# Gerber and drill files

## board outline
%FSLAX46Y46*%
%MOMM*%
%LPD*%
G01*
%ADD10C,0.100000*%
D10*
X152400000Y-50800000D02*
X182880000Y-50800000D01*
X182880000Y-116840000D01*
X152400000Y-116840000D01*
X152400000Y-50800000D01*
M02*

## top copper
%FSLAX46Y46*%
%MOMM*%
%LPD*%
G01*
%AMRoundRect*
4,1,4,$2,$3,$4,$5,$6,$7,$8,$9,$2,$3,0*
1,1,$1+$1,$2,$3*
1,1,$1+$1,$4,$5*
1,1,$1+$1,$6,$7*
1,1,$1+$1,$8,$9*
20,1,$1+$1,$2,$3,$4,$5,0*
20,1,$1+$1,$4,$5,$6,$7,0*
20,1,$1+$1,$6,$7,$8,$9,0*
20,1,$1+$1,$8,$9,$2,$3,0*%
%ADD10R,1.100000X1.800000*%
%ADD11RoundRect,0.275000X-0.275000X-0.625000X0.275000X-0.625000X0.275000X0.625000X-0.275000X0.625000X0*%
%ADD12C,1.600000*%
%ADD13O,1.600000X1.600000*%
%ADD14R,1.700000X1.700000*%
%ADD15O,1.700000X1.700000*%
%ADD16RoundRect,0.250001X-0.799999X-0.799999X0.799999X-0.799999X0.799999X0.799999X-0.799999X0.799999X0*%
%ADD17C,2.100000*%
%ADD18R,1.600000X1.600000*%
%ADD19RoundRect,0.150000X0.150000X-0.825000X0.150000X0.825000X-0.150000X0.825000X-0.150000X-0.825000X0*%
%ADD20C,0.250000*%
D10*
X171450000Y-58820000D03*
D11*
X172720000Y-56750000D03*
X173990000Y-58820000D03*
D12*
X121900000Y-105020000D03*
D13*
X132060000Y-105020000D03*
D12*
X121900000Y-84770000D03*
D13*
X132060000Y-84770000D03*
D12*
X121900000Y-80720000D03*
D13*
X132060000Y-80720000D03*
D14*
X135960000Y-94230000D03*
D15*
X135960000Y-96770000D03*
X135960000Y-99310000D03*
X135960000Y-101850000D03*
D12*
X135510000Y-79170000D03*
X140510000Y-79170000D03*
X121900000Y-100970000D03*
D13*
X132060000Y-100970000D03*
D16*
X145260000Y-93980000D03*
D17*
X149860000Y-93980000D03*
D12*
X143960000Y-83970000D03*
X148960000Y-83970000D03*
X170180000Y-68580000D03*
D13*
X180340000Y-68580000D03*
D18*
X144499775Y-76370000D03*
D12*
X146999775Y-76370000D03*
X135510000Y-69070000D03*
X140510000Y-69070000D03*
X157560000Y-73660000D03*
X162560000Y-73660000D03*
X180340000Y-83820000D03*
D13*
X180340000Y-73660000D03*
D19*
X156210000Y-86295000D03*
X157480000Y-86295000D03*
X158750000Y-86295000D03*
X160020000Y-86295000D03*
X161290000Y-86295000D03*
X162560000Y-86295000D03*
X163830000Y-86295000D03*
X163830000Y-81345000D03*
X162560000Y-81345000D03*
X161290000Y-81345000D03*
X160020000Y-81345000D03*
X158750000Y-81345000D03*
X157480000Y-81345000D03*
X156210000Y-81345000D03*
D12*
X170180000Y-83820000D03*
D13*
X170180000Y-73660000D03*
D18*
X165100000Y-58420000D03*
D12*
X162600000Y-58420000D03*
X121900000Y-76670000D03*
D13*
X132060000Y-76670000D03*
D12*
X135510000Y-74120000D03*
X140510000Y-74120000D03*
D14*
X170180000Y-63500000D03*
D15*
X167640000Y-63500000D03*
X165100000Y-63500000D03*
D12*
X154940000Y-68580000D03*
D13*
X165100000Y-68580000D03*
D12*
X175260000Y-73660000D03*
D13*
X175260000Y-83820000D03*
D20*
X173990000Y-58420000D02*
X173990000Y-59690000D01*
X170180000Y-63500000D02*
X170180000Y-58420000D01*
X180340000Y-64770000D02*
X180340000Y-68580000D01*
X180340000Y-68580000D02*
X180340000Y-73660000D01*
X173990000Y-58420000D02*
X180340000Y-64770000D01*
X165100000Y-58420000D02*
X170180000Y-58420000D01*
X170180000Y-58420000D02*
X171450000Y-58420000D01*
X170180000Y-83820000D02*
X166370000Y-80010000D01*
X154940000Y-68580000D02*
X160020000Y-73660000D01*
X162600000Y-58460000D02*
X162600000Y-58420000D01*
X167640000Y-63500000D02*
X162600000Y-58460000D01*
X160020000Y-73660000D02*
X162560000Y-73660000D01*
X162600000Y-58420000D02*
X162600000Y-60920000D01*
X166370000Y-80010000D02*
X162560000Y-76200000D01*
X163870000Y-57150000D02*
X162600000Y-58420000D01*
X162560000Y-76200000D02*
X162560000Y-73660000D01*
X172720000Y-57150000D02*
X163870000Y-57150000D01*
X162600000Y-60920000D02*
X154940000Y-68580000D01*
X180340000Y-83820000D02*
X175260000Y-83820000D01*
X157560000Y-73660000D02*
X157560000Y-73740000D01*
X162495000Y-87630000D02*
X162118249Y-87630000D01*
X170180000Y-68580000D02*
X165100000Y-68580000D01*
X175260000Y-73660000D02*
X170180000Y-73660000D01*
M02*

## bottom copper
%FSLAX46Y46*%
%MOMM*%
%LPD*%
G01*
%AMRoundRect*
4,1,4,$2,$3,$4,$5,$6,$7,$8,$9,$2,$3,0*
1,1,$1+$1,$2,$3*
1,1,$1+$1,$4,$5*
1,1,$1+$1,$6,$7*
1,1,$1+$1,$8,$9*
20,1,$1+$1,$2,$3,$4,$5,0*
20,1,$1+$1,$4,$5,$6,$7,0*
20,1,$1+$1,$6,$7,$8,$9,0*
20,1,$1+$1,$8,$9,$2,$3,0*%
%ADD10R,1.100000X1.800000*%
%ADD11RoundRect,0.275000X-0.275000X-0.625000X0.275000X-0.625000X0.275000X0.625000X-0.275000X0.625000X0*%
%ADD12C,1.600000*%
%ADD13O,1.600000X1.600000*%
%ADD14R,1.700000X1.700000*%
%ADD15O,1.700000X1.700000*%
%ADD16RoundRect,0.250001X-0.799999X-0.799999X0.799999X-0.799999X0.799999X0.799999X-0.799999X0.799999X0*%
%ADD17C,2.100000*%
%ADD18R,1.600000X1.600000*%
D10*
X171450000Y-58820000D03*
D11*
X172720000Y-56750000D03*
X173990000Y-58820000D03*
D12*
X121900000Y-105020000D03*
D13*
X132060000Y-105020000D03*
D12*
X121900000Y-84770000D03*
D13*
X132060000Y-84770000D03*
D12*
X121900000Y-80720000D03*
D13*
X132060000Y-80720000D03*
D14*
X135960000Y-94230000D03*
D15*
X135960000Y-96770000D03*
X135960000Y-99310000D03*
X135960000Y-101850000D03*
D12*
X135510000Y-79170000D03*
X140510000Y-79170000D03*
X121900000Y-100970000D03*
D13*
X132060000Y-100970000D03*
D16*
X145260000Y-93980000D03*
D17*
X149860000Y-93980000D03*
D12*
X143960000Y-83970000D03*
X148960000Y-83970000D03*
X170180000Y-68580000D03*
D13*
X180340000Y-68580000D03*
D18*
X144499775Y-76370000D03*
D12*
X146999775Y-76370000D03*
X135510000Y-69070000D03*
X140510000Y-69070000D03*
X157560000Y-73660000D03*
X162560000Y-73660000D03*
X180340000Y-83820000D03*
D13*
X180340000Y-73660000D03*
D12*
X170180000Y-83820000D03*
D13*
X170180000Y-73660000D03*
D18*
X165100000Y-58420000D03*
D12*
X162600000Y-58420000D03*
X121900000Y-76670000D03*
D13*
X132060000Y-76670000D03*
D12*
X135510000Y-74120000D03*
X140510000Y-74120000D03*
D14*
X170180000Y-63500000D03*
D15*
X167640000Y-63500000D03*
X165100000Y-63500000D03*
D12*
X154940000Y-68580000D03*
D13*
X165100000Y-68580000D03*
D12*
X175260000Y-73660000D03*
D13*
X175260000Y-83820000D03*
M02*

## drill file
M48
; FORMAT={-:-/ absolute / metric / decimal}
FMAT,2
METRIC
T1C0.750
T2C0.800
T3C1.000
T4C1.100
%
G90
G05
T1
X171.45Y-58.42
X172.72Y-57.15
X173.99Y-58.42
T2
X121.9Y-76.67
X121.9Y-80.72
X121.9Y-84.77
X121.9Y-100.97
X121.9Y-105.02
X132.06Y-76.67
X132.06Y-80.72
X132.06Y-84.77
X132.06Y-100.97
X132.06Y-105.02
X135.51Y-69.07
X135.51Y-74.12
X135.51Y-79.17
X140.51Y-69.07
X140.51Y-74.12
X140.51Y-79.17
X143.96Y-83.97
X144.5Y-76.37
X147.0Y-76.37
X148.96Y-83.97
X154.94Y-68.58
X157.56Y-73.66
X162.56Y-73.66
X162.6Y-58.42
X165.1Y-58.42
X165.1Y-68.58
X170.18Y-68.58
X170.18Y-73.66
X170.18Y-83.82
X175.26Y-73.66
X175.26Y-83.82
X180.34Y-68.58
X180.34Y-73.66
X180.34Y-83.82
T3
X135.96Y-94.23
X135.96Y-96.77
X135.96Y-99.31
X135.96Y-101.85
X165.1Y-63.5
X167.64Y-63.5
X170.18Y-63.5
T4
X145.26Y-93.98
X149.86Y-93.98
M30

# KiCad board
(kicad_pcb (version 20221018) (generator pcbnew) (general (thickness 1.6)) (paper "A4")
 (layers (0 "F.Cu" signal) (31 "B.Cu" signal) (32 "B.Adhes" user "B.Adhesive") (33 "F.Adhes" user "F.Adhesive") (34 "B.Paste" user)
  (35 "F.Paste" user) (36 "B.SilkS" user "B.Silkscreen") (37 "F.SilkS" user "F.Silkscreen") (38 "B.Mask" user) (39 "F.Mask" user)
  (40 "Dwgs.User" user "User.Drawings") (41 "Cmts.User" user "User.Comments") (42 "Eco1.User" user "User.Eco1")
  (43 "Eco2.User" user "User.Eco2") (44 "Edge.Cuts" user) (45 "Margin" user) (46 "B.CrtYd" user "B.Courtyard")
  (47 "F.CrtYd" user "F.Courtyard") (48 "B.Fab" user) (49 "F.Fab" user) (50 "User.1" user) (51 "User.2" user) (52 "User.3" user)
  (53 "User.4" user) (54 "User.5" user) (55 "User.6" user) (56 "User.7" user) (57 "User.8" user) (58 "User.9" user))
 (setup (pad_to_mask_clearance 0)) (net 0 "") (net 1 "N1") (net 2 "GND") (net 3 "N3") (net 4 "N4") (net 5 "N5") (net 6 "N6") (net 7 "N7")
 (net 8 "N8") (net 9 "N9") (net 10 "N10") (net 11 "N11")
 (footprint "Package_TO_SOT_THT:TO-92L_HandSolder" (layer "F.Cu") (at 171.45 58.42)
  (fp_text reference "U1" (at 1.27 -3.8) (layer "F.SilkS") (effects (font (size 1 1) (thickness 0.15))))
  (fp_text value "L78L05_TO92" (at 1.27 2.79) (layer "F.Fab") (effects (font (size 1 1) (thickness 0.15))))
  (pad "1" thru_hole rect (at 0 0) (size 1.1 1.8) (drill 0.75 (offset 0 0.4)) (layers "*.Cu" "*.Mask") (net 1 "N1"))
  (pad "2" thru_hole roundrect (at 1.27 -1.27) (size 1.1 1.8) (drill 0.75 (offset 0 -0.4)) (layers "*.Cu" "*.Mask") (roundrect_rratio 0.25)
   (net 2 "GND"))
  (pad "3" thru_hole roundrect (at 2.54 0) (size 1.1 1.8) (drill 0.75 (offset 0 0.4)) (layers "*.Cu" "*.Mask") (roundrect_rratio 0.25)
   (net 1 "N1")))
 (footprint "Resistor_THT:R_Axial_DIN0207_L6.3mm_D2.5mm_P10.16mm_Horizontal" (layer "F.Cu") (at 121.9 105.02)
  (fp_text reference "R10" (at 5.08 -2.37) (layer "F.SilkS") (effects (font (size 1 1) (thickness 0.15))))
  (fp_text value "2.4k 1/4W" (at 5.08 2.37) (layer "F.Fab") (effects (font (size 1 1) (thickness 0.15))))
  (pad "1" thru_hole circle (at 0 0) (size 1.6 1.6) (drill 0.8) (layers "*.Cu" "*.Mask") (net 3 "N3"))
  (pad "2" thru_hole oval (at 10.16 0) (size 1.6 1.6) (drill 0.8) (layers "*.Cu" "*.Mask") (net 1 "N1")))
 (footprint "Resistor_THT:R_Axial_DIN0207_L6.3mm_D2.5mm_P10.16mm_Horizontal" (layer "F.Cu") (at 121.9 84.77)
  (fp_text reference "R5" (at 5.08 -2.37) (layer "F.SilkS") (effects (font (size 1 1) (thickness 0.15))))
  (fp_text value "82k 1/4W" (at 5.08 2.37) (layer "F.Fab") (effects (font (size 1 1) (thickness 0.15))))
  (pad "1" thru_hole circle (at 0 0) (size 1.6 1.6) (drill 0.8) (layers "*.Cu" "*.Mask") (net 2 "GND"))
  (pad "2" thru_hole oval (at 10.16 0) (size 1.6 1.6) (drill 0.8) (layers "*.Cu" "*.Mask") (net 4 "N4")))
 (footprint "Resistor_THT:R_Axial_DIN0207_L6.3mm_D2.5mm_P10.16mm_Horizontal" (layer "F.Cu") (at 121.9 80.72)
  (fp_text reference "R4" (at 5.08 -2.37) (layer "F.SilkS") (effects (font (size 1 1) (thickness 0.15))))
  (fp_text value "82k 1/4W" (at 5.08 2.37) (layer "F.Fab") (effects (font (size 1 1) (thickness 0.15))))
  (pad "1" thru_hole circle (at 0 0) (size 1.6 1.6) (drill 0.8) (layers "*.Cu" "*.Mask") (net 4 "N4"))
  (pad "2" thru_hole oval (at 10.16 0) (size 1.6 1.6) (drill 0.8) (layers "*.Cu" "*.Mask") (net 1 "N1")))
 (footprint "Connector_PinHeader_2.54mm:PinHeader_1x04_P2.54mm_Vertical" (layer "F.Cu") (at 135.96 94.23)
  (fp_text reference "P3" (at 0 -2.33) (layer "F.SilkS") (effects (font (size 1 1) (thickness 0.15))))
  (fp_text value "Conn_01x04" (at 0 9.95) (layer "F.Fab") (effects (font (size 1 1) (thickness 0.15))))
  (pad "1" thru_hole rect (at 0 0) (size 1.7 1.7) (drill 1) (layers "*.Cu" "*.Mask") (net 1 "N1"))
  (pad "2" thru_hole oval (at 0 2.54) (size 1.7 1.7) (drill 1) (layers "*.Cu" "*.Mask") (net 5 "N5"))
  (pad "3" thru_hole oval (at 0 5.08) (size 1.7 1.7) (drill 1) (layers "*.Cu" "*.Mask") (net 3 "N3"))
  (pad "4" thru_hole oval (at 0 7.62) (size 1.7 1.7) (drill 1) (layers "*.Cu" "*.Mask") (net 2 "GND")))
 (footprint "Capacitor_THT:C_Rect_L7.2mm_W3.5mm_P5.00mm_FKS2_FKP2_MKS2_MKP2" (layer "F.Cu") (at 135.51 79.17)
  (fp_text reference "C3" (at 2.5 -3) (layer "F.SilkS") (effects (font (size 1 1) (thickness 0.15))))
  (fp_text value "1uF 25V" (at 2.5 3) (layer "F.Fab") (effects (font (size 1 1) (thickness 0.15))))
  (pad "1" thru_hole circle (at 0 0) (size 1.6 1.6) (drill 0.8) (layers "*.Cu" "*.Mask") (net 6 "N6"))
  (pad "2" thru_hole circle (at 5 0) (size 1.6 1.6) (drill 0.8) (layers "*.Cu" "*.Mask") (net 4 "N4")))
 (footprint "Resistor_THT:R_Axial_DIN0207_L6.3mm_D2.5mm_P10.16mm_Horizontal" (layer "F.Cu") (at 121.9 100.97)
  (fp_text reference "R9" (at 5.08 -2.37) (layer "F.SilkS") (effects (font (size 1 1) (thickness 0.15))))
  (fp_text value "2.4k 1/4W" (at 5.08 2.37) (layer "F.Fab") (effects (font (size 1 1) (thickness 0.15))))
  (pad "1" thru_hole circle (at 0 0) (size 1.6 1.6) (drill 0.8) (layers "*.Cu" "*.Mask") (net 5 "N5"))
  (pad "2" thru_hole oval (at 10.16 0) (size 1.6 1.6) (drill 0.8) (layers "*.Cu" "*.Mask") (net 1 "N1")))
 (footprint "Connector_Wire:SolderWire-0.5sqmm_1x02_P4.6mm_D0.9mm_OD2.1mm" (layer "F.Cu") (at 145.26 93.98)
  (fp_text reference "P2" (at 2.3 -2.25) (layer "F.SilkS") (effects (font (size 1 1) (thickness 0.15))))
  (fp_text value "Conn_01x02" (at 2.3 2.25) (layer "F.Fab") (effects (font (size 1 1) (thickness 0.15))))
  (pad "1" thru_hole roundrect (at 0 0) (size 2.1 2.1) (drill 1.1) (layers "*.Cu" "*.Mask") (roundrect_rratio 0.119048) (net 1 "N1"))
  (pad "2" thru_hole circle (at 4.6 0) (size 2.1 2.1) (drill 1.1) (layers "*.Cu" "*.Mask") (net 2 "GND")))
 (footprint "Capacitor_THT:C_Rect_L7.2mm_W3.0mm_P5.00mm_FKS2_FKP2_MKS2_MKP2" (layer "F.Cu") (at 143.96 83.97)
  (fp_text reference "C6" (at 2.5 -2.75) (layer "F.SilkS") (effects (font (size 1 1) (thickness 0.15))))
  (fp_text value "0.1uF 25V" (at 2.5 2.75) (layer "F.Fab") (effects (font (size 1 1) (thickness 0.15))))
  (pad "1" thru_hole circle (at 0 0) (size 1.6 1.6) (drill 0.8) (layers "*.Cu" "*.Mask") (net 1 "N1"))
  (pad "2" thru_hole circle (at 5 0) (size 1.6 1.6) (drill 0.8) (layers "*.Cu" "*.Mask") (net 2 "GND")))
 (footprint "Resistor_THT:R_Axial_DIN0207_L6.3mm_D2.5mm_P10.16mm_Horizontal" (layer "F.Cu") (at 170.18 68.58)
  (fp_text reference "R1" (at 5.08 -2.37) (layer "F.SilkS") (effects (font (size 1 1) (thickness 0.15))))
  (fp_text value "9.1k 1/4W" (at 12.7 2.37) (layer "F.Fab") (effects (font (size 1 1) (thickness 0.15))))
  (pad "1" thru_hole circle (at 0 0) (size 1.6 1.6) (drill 0.8) (layers "*.Cu" "*.Mask") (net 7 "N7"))
  (pad "2" thru_hole oval (at 10.16 0) (size 1.6 1.6) (drill 0.8) (layers "*.Cu" "*.Mask") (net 1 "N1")))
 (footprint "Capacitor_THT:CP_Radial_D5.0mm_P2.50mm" (layer "F.Cu") (at 144.499775 76.37)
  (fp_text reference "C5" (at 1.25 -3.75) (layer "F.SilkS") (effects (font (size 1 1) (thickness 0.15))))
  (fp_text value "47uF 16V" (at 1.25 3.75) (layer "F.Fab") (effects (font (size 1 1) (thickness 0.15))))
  (pad "1" thru_hole rect (at 0 0) (size 1.6 1.6) (drill 0.8) (layers "*.Cu" "*.Mask") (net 1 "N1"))
  (pad "2" thru_hole circle (at 2.5 0) (size 1.6 1.6) (drill 0.8) (layers "*.Cu" "*.Mask") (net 2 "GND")))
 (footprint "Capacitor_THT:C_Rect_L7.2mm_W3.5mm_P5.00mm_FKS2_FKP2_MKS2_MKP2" (layer "F.Cu") (at 135.51 69.07)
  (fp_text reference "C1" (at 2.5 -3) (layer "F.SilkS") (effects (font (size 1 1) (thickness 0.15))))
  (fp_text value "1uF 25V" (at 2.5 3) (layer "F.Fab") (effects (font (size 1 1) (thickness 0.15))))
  (pad "1" thru_hole circle (at 0 0) (size 1.6 1.6) (drill 0.8) (layers "*.Cu" "*.Mask") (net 6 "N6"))
  (pad "2" thru_hole circle (at 5 0) (size 1.6 1.6) (drill 0.8) (layers "*.Cu" "*.Mask") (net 4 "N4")))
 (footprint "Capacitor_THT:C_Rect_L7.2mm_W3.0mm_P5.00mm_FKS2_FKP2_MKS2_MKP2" (layer "F.Cu") (at 157.56 73.66)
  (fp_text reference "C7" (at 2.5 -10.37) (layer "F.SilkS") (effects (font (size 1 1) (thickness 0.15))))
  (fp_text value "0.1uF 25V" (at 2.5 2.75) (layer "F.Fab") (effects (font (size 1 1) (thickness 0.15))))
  (pad "1" thru_hole circle (at 0 0) (size 1.6 1.6) (drill 0.8) (layers "*.Cu" "*.Mask") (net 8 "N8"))
  (pad "2" thru_hole circle (at 5 0) (size 1.6 1.6) (drill 0.8) (layers "*.Cu" "*.Mask") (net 2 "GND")))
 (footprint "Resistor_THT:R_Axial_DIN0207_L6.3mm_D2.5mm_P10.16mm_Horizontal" (layer "F.Cu") (at 180.34 83.82 90)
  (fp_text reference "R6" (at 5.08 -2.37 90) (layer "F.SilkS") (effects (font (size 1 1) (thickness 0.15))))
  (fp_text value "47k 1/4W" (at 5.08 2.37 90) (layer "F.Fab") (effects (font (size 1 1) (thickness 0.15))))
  (pad "1" thru_hole circle (at 0 0 90) (size 1.6 1.6) (drill 0.8) (layers "*.Cu" "*.Mask") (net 8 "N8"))
  (pad "2" thru_hole oval (at 10.16 0 90) (size 1.6 1.6) (drill 0.8) (layers "*.Cu" "*.Mask") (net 1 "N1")))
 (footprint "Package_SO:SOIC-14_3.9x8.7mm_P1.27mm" (layer "F.Cu") (at 160.02 83.82 90)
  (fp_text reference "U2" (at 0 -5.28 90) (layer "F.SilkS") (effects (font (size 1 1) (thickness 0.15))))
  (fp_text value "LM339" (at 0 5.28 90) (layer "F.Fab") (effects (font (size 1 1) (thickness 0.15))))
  (pad "1" smd roundrect (at -2.475 -3.81 90) (size 1.95 0.6) (layers "F.Cu" "F.Paste" "F.Mask") (roundrect_rratio 0.25) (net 3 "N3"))
  (pad "2" smd roundrect (at -2.475 -2.54 90) (size 1.95 0.6) (layers "F.Cu" "F.Paste" "F.Mask") (roundrect_rratio 0.25) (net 5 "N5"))
  (pad "3" smd roundrect (at -2.475 -1.27 90) (size 1.95 0.6) (layers "F.Cu" "F.Paste" "F.Mask") (roundrect_rratio 0.25) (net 1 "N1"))
  (pad "4" smd roundrect (at -2.475 0 90) (size 1.95 0.6) (layers "F.Cu" "F.Paste" "F.Mask") (roundrect_rratio 0.25) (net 8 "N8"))
  (pad "5" smd roundrect (at -2.475 1.27 90) (size 1.95 0.6) (layers "F.Cu" "F.Paste" "F.Mask") (roundrect_rratio 0.25) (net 4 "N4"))
  (pad "6" smd roundrect (at -2.475 2.54 90) (size 1.95 0.6) (layers "F.Cu" "F.Paste" "F.Mask") (roundrect_rratio 0.25) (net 4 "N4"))
  (pad "7" smd roundrect (at -2.475 3.81 90) (size 1.95 0.6) (layers "F.Cu" "F.Paste" "F.Mask") (roundrect_rratio 0.25) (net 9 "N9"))
  (pad "8" smd roundrect (at 2.475 3.81 90) (size 1.95 0.6) (layers "F.Cu" "F.Paste" "F.Mask") (roundrect_rratio 0.25) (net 7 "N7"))
  (pad "9" smd roundrect (at 2.475 2.54 90) (size 1.95 0.6) (layers "F.Cu" "F.Paste" "F.Mask") (roundrect_rratio 0.25) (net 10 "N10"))
  (pad "10" smd roundrect (at 2.475 1.27 90) (size 1.95 0.6) (layers "F.Cu" "F.Paste" "F.Mask") (roundrect_rratio 0.25) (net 9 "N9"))
  (pad "11" smd roundrect (at 2.475 0 90) (size 1.95 0.6) (layers "F.Cu" "F.Paste" "F.Mask") (roundrect_rratio 0.25) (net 7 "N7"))
  (pad "12" smd roundrect (at 2.475 -1.27 90) (size 1.95 0.6) (layers "F.Cu" "F.Paste" "F.Mask") (roundrect_rratio 0.25) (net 2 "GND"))
  (pad "13" smd roundrect (at 2.475 -2.54 90) (size 1.95 0.6) (layers "F.Cu" "F.Paste" "F.Mask") (roundrect_rratio 0.25) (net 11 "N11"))
  (pad "14" smd roundrect (at 2.475 -3.81 90) (size 1.95 0.6) (layers "F.Cu" "F.Paste" "F.Mask") (roundrect_rratio 0.25) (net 6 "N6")))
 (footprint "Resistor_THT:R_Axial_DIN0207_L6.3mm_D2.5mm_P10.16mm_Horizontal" (layer "F.Cu") (at 170.18 83.82 90)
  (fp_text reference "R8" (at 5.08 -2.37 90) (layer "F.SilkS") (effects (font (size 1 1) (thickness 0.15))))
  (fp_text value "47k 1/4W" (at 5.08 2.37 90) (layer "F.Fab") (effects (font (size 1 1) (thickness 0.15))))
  (pad "1" thru_hole circle (at 0 0 90) (size 1.6 1.6) (drill 0.8) (layers "*.Cu" "*.Mask") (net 2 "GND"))
  (pad "2" thru_hole oval (at 10.16 0 90) (size 1.6 1.6) (drill 0.8) (layers "*.Cu" "*.Mask") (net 9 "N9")))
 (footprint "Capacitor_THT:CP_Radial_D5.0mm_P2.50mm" (layer "F.Cu") (at 165.1 58.42 180)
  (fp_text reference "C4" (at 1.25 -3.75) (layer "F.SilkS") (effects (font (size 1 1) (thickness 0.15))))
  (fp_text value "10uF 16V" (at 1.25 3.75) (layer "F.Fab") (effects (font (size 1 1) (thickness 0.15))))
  (pad "1" thru_hole rect (at 0 0 180) (size 1.6 1.6) (drill 0.8) (layers "*.Cu" "*.Mask") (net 1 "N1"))
  (pad "2" thru_hole circle (at 2.5 0 180) (size 1.6 1.6) (drill 0.8) (layers "*.Cu" "*.Mask") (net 2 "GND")))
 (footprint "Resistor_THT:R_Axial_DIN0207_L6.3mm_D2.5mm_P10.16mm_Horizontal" (layer "F.Cu") (at 121.9 76.67)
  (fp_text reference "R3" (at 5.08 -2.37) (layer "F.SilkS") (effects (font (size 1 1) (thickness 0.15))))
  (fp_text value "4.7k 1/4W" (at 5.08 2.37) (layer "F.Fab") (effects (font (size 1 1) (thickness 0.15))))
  (pad "1" thru_hole circle (at 0 0) (size 1.6 1.6) (drill 0.8) (layers "*.Cu" "*.Mask") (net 6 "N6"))
  (pad "2" thru_hole oval (at 10.16 0) (size 1.6 1.6) (drill 0.8) (layers "*.Cu" "*.Mask") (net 1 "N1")))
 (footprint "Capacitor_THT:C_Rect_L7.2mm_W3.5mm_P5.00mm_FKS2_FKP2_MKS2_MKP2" (layer "F.Cu") (at 135.51 74.12)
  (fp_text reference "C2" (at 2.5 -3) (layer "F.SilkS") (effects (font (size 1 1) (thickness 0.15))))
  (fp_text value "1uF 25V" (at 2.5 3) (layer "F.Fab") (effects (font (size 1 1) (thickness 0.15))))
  (pad "1" thru_hole circle (at 0 0) (size 1.6 1.6) (drill 0.8) (layers "*.Cu" "*.Mask") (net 6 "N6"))
  (pad "2" thru_hole circle (at 5 0) (size 1.6 1.6) (drill 0.8) (layers "*.Cu" "*.Mask") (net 4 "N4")))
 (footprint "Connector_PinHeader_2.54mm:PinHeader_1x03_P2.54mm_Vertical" (layer "F.Cu") (at 170.18 63.5 -90)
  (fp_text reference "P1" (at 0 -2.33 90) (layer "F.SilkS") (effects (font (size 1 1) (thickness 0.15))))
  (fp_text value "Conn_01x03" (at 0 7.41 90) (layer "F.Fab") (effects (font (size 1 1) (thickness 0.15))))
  (pad "1" thru_hole rect (at 0 0 270) (size 1.7 1.7) (drill 1) (layers "*.Cu" "*.Mask") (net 1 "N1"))
  (pad "2" thru_hole oval (at 0 2.54 270) (size 1.7 1.7) (drill 1) (layers "*.Cu" "*.Mask") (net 2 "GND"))
  (pad "3" thru_hole oval (at 0 5.08 270) (size 1.7 1.7) (drill 1) (layers "*.Cu" "*.Mask") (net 10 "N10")))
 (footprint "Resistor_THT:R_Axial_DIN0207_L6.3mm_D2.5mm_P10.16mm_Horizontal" (layer "F.Cu") (at 154.94 68.58)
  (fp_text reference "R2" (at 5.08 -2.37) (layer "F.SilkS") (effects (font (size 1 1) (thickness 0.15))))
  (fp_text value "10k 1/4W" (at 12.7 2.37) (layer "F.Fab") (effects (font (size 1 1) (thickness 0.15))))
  (pad "1" thru_hole circle (at 0 0) (size 1.6 1.6) (drill 0.8) (layers "*.Cu" "*.Mask") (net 2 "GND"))
  (pad "2" thru_hole oval (at 10.16 0) (size 1.6 1.6) (drill 0.8) (layers "*.Cu" "*.Mask") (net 7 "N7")))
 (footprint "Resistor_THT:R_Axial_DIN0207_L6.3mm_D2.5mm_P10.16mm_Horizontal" (layer "F.Cu") (at 175.26 73.66 -90)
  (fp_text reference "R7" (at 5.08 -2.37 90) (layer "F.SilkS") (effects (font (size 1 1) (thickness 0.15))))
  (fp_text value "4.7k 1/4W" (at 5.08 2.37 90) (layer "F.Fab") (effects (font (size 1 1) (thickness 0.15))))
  (pad "1" thru_hole circle (at 0 0 270) (size 1.6 1.6) (drill 0.8) (layers "*.Cu" "*.Mask") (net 9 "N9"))
  (pad "2" thru_hole oval (at 10.16 0 270) (size 1.6 1.6) (drill 0.8) (layers "*.Cu" "*.Mask") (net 8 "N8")))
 (gr_rect (start 152.4 50.8) (end 182.88 116.84) (stroke (width 0.1) (type default)) (fill none) (layer "Edge.Cuts"))
 (segment (start 173.99 58.42) (end 173.99 59.69) (width 0.25) (layer "F.Cu") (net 1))
 (segment (start 170.18 63.5) (end 170.18 58.42) (width 0.25) (layer "F.Cu") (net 1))
 (segment (start 180.34 64.77) (end 180.34 68.58) (width 0.25) (layer "F.Cu") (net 1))
 (segment (start 180.34 68.58) (end 180.34 73.66) (width 0.25) (layer "F.Cu") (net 1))
 (segment (start 173.99 58.42) (end 180.34 64.77) (width 0.25) (layer "F.Cu") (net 1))
 (segment (start 165.1 58.42) (end 170.18 58.42) (width 0.25) (layer "F.Cu") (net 1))
 (segment (start 170.18 58.42) (end 171.45 58.42) (width 0.25) (layer "F.Cu") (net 1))
 (segment (start 170.18 83.82) (end 166.37 80.01) (width 0.25) (layer "F.Cu") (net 2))
 (segment (start 154.94 68.58) (end 160.02 73.66) (width 0.25) (layer "F.Cu") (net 2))
 (segment (start 162.6 58.46) (end 162.6 58.42) (width 0.25) (layer "F.Cu") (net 2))
 (segment (start 167.64 63.5) (end 162.6 58.46) (width 0.25) (layer "F.Cu") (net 2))
 (segment (start 160.02 73.66) (end 162.56 73.66) (width 0.25) (layer "F.Cu") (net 2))
 (segment (start 162.6 58.42) (end 162.6 60.92) (width 0.25) (layer "F.Cu") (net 2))
 (segment (start 166.37 80.01) (end 162.56 76.2) (width 0.25) (layer "F.Cu") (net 2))
 (segment (start 163.87 57.15) (end 162.6 58.42) (width 0.25) (layer "F.Cu") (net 2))
 (segment (start 162.56 76.2) (end 162.56 73.66) (width 0.25) (layer "F.Cu") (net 2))
 (segment (start 172.72 57.15) (end 163.87 57.15) (width 0.25) (layer "F.Cu") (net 2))
 (segment (start 162.6 60.92) (end 154.94 68.58) (width 0.25) (layer "F.Cu") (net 2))
 (segment (start 180.34 83.82) (end 175.26 83.82) (width 0.25) (layer "F.Cu") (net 8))
 (segment (start 157.56 73.66) (end 157.56 73.74) (width 0.25) (layer "F.Cu") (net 8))
 (segment (start 162.495 87.63) (end 162.118249 87.63) (width 0.25) (layer "F.Cu") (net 3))
 (segment (start 170.18 68.58) (end 165.1 68.58) (width 0.25) (layer "F.Cu") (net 7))
 (segment (start 175.26 73.66) (end 170.18 73.66) (width 0.25) (layer "F.Cu") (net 9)))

